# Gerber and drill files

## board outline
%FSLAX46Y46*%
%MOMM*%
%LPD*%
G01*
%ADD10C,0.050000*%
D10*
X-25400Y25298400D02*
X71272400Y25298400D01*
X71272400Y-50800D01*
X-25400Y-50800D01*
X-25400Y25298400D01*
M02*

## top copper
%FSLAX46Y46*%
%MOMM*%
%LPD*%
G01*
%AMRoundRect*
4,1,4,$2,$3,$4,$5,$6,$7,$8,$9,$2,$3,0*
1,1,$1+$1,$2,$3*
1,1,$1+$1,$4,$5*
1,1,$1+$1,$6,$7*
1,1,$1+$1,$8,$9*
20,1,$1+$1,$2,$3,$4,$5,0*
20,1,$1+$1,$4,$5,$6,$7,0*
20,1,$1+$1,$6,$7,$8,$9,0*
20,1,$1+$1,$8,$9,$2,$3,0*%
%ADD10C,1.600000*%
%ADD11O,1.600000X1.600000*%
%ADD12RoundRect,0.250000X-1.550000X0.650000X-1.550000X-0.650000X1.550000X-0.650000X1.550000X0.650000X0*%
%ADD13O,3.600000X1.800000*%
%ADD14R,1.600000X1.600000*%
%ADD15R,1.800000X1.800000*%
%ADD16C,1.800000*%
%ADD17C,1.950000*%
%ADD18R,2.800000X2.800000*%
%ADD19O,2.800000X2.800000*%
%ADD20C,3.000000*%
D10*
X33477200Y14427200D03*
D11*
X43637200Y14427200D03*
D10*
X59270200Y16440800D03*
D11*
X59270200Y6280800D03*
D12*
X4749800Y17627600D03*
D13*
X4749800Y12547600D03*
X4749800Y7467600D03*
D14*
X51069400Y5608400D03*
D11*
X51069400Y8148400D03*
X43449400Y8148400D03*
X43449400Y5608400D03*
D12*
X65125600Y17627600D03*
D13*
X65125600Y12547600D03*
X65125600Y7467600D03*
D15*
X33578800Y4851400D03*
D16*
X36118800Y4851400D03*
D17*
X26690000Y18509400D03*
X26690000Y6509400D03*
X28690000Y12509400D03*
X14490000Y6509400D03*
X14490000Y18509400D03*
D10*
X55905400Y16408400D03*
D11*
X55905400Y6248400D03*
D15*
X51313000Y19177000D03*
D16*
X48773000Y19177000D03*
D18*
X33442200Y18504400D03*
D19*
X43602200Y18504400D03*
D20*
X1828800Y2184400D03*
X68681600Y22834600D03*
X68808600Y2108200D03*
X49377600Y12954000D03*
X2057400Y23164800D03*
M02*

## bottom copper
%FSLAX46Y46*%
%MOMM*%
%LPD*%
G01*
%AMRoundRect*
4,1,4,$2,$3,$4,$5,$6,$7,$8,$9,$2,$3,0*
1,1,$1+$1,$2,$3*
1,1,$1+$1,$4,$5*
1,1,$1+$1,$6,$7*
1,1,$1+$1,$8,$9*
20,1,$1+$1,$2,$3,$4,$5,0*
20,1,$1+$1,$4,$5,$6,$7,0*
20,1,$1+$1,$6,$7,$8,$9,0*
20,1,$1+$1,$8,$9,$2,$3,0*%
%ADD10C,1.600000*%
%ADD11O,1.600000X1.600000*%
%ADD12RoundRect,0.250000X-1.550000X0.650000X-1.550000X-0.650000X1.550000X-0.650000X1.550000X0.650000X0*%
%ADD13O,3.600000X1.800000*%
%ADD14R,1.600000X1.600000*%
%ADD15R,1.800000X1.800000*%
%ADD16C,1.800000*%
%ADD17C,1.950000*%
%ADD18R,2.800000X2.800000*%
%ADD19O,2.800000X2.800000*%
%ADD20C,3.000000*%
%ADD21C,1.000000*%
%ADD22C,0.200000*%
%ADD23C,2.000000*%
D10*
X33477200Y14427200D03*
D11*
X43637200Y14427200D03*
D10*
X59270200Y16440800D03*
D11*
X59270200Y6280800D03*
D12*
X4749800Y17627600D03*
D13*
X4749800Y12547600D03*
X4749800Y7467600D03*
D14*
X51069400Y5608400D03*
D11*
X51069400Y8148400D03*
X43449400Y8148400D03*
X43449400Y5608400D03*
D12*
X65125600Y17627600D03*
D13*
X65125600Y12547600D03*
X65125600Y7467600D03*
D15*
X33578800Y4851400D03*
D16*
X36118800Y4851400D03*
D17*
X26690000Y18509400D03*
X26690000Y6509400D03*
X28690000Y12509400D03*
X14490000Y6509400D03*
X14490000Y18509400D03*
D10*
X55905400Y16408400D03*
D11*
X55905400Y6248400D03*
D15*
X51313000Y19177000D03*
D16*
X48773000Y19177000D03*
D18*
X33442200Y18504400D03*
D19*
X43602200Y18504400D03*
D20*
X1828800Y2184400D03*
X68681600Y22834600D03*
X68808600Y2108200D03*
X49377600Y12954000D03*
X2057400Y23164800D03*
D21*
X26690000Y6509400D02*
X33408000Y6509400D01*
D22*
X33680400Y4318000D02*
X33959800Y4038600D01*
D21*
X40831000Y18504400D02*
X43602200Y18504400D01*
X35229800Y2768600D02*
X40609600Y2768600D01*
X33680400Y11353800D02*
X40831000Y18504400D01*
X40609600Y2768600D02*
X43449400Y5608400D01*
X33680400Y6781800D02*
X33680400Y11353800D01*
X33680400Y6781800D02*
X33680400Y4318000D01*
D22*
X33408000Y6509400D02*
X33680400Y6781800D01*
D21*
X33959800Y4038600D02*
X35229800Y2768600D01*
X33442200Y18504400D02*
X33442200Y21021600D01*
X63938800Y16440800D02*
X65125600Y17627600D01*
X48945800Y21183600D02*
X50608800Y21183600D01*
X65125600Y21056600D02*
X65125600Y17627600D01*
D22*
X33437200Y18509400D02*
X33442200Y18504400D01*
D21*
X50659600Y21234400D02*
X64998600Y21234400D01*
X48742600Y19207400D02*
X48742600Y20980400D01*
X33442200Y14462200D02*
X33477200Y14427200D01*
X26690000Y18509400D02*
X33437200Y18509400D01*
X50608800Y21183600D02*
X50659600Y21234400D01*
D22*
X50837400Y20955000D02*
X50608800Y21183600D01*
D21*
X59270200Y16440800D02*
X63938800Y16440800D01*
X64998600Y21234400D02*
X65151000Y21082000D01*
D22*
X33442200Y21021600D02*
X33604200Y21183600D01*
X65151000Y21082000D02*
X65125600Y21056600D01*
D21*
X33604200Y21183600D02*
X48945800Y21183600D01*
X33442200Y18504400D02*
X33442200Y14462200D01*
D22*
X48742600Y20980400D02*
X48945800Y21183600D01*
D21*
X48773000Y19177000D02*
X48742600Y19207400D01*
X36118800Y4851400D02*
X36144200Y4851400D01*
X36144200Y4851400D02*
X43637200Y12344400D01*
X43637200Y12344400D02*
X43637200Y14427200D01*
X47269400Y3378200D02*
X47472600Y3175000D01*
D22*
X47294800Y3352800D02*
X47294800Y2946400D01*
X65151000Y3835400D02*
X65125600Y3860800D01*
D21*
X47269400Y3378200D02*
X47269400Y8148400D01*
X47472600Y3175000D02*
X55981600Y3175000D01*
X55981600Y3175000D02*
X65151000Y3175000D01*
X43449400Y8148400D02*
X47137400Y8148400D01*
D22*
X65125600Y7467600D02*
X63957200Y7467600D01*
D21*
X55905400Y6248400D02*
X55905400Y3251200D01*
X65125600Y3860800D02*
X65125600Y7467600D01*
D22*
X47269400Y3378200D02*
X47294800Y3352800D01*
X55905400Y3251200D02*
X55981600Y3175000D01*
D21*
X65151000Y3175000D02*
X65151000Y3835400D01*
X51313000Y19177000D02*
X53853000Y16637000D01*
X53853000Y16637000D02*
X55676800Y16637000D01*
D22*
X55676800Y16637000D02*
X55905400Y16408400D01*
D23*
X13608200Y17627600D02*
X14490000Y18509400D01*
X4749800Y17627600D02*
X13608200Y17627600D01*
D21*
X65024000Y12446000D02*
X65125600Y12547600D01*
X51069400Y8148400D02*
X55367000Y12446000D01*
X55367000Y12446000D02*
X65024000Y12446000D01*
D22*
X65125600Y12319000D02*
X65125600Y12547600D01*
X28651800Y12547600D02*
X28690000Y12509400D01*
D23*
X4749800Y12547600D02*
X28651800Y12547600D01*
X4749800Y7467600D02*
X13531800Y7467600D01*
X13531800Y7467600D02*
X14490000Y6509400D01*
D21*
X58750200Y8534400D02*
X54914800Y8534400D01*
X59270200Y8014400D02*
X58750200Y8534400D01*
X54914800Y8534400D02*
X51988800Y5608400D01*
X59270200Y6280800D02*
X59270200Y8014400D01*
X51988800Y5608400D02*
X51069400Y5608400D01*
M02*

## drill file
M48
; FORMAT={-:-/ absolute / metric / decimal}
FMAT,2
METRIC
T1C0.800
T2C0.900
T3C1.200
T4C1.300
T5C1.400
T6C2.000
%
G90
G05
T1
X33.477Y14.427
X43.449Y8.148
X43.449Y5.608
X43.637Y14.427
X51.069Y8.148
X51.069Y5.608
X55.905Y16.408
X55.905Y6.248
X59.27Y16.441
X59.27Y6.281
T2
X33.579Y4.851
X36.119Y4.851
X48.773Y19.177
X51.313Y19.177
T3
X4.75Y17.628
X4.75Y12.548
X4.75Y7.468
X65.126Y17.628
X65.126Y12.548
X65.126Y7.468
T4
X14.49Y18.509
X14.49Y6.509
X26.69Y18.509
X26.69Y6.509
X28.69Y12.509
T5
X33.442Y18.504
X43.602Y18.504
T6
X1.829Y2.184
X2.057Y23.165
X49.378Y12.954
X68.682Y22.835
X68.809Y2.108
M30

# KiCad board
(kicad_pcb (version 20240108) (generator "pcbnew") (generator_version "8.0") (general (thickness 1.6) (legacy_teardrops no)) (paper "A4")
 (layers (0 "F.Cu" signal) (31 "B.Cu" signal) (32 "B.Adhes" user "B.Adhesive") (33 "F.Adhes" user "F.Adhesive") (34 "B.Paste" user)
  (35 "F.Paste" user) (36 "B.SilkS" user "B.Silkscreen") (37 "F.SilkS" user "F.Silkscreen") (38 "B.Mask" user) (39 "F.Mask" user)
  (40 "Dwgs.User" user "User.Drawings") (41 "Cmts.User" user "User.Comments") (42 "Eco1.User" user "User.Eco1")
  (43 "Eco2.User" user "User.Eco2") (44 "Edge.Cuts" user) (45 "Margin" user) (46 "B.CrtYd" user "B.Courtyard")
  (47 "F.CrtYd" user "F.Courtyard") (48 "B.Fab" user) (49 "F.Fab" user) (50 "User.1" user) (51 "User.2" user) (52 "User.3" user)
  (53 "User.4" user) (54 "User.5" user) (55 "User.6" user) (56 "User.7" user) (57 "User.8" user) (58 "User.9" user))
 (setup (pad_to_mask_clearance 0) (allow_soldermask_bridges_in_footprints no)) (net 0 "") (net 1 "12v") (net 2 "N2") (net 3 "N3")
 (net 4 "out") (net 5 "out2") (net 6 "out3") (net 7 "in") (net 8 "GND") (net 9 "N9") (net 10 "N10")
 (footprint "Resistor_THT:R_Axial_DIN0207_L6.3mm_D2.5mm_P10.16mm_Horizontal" (layer "F.Cu") (at 33.4772 -14.4272)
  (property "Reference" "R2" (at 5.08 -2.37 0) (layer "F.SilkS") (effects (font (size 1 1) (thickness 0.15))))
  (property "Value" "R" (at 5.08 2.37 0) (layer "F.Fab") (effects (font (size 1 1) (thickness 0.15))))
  (pad "1" thru_hole circle (at 0 0) (size 1.6 1.6) (drill 0.8) (layers "*.Cu" "*.Mask") (remove_unused_layers no) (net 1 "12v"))
  (pad "2" thru_hole oval (at 10.16 0) (size 1.6 1.6) (drill 0.8) (layers "*.Cu" "*.Mask") (remove_unused_layers no) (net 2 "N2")))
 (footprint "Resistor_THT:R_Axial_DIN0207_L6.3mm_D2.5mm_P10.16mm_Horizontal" (layer "F.Cu") (at 59.2702 -16.4408 -90)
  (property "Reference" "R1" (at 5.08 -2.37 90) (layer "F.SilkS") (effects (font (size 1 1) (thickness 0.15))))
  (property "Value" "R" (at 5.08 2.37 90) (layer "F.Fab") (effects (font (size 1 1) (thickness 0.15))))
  (pad "1" thru_hole circle (at 0 0 270) (size 1.6 1.6) (drill 0.8) (layers "*.Cu" "*.Mask") (remove_unused_layers no) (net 1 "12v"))
  (pad "2" thru_hole oval (at 10.16 0 270) (size 1.6 1.6) (drill 0.8) (layers "*.Cu" "*.Mask") (remove_unused_layers no) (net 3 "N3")))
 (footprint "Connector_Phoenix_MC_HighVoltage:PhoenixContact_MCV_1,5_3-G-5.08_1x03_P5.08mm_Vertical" (layer "F.Cu") (at 4.7498 -17.6276 -90)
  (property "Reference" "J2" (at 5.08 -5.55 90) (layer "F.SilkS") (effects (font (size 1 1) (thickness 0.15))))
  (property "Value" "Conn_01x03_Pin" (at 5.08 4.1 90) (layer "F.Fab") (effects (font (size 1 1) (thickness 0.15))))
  (pad "1" thru_hole roundrect (at 0 0 270) (size 1.8 3.6) (drill 1.2) (layers "*.Cu" "*.Mask") (remove_unused_layers no)
   (roundrect_rratio 0.138889) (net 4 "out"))
  (pad "2" thru_hole oval (at 5.08 0 270) (size 1.8 3.6) (drill 1.2) (layers "*.Cu" "*.Mask") (remove_unused_layers no) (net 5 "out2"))
  (pad "3" thru_hole oval (at 10.16 0 270) (size 1.8 3.6) (drill 1.2) (layers "*.Cu" "*.Mask") (remove_unused_layers no) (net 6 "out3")))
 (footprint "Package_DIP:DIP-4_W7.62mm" (layer "F.Cu") (at 51.0694 -5.6084 180)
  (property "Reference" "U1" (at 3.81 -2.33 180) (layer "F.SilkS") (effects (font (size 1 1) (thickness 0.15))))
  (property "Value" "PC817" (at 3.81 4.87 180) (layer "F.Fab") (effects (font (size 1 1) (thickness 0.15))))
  (pad "1" thru_hole rect (at 0 0 180) (size 1.6 1.6) (drill 0.8) (layers "*.Cu" "*.Mask") (remove_unused_layers no) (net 3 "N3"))
  (pad "2" thru_hole oval (at 0 2.54 180) (size 1.6 1.6) (drill 0.8) (layers "*.Cu" "*.Mask") (remove_unused_layers no) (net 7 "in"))
  (pad "3" thru_hole oval (at 7.62 2.54 180) (size 1.6 1.6) (drill 0.8) (layers "*.Cu" "*.Mask") (remove_unused_layers no) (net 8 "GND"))
  (pad "4" thru_hole oval (at 7.62 0 180) (size 1.6 1.6) (drill 0.8) (layers "*.Cu" "*.Mask") (remove_unused_layers no) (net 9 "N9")))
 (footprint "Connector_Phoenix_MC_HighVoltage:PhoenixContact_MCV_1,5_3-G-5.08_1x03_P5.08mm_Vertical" (layer "F.Cu")
  (at 65.1256 -17.6276 -90)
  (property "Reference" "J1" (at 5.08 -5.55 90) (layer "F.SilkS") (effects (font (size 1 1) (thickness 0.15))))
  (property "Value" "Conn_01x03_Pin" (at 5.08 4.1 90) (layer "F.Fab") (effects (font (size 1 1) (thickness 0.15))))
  (pad "1" thru_hole roundrect (at 0 0 270) (size 1.8 3.6) (drill 1.2) (layers "*.Cu" "*.Mask") (remove_unused_layers no)
   (roundrect_rratio 0.138889) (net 1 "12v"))
  (pad "2" thru_hole oval (at 5.08 0 270) (size 1.8 3.6) (drill 1.2) (layers "*.Cu" "*.Mask") (remove_unused_layers no) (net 7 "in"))
  (pad "3" thru_hole oval (at 10.16 0 270) (size 1.8 3.6) (drill 1.2) (layers "*.Cu" "*.Mask") (remove_unused_layers no) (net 8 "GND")))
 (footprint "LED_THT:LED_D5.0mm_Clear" (layer "F.Cu") (at 33.5788 -4.8514)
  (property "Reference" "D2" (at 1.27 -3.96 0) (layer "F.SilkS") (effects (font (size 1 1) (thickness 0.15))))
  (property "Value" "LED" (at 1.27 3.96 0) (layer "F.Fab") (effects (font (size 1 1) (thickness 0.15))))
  (pad "1" thru_hole rect (at 0 0) (size 1.8 1.8) (drill 0.9) (layers "*.Cu" "*.Mask") (remove_unused_layers no) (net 9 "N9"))
  (pad "2" thru_hole circle (at 2.54 0) (size 1.8 1.8) (drill 0.9) (layers "*.Cu" "*.Mask") (remove_unused_layers no) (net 2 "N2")))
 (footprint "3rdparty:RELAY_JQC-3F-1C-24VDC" (layer "F.Cu") (at 20.59 -12.5094)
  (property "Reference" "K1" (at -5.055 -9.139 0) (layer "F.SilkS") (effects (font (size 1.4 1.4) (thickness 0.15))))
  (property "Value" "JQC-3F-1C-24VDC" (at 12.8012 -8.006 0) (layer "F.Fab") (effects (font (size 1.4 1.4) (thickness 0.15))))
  (pad "COIL1" thru_hole circle (at 6.1 -6) (size 1.95 1.95) (drill 1.3) (layers "*.Cu" "*.Mask") (remove_unused_layers no) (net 1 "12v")
   (solder_mask_margin 0.102))
  (pad "COIL2" thru_hole circle (at 6.1 6) (size 1.95 1.95) (drill 1.3) (layers "*.Cu" "*.Mask") (remove_unused_layers no) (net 9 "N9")
   (solder_mask_margin 0.102))
  (pad "COM" thru_hole circle (at 8.1 0) (size 1.95 1.95) (drill 1.3) (layers "*.Cu" "*.Mask") (remove_unused_layers no) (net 5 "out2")
   (solder_mask_margin 0.102))
  (pad "NC" thru_hole circle (at -6.1 6) (size 1.95 1.95) (drill 1.3) (layers "*.Cu" "*.Mask") (remove_unused_layers no) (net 6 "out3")
   (solder_mask_margin 0.102))
  (pad "NO" thru_hole circle (at -6.1 -6) (size 1.95 1.95) (drill 1.3) (layers "*.Cu" "*.Mask") (remove_unused_layers no) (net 4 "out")
   (solder_mask_margin 0.102)))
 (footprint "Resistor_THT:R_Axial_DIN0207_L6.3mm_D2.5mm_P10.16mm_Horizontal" (layer "F.Cu") (at 55.9054 -16.4084 -90)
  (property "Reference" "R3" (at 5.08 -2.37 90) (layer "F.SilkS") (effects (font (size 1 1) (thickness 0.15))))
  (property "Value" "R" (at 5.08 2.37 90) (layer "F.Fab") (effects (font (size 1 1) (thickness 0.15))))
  (pad "1" thru_hole circle (at 0 0 270) (size 1.6 1.6) (drill 0.8) (layers "*.Cu" "*.Mask") (remove_unused_layers no) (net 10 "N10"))
  (pad "2" thru_hole oval (at 10.16 0 270) (size 1.6 1.6) (drill 0.8) (layers "*.Cu" "*.Mask") (remove_unused_layers no) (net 8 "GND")))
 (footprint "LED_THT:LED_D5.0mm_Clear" (layer "F.Cu") (at 51.313 -19.177 180)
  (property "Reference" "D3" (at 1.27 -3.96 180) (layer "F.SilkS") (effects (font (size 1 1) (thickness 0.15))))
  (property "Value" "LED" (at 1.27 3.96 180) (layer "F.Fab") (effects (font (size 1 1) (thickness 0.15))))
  (pad "1" thru_hole rect (at 0 0 180) (size 1.8 1.8) (drill 0.9) (layers "*.Cu" "*.Mask") (remove_unused_layers no) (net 10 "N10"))
  (pad "2" thru_hole circle (at 2.54 0 180) (size 1.8 1.8) (drill 0.9) (layers "*.Cu" "*.Mask") (remove_unused_layers no) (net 1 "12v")))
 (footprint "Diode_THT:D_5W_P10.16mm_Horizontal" (layer "F.Cu") (at 33.4422 -18.5044)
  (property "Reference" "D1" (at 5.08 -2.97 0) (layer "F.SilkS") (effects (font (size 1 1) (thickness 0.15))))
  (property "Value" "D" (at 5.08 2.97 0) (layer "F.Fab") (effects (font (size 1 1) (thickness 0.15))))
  (pad "1" thru_hole rect (at 0 0) (size 2.8 2.8) (drill 1.4) (layers "*.Cu" "*.Mask") (remove_unused_layers no) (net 1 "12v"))
  (pad "2" thru_hole oval (at 10.16 0) (size 2.8 2.8) (drill 1.4) (layers "*.Cu" "*.Mask") (remove_unused_layers no) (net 9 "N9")))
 (gr_rect (start -0.0254 -25.2984) (end 71.2724 0.0508) (stroke (width 0.05) (type default)) (fill none) (layer "Edge.Cuts"))
 (via (at 1.8288 -2.1844) (size 3) (drill 2) (layers "F.Cu" "B.Cu") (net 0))
 (via (at 68.6816 -22.8346) (size 3) (drill 2) (layers "F.Cu" "B.Cu") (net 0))
 (via (at 68.8086 -2.1082) (size 3) (drill 2) (layers "F.Cu" "B.Cu") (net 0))
 (via (at 49.3776 -12.954) (size 3) (drill 2) (layers "F.Cu" "B.Cu") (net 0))
 (via (at 2.0574 -23.1648) (size 3) (drill 2) (layers "F.Cu" "B.Cu") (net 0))
 (segment (start 26.69 -6.5094) (end 33.408 -6.5094) (width 1) (layer "B.Cu") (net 9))
 (segment (start 33.6804 -4.318) (end 33.9598 -4.0386) (width 0.2) (layer "B.Cu") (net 9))
 (segment (start 40.831 -18.5044) (end 43.6022 -18.5044) (width 1) (layer "B.Cu") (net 9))
 (segment (start 35.2298 -2.7686) (end 40.6096 -2.7686) (width 1) (layer "B.Cu") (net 9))
 (segment (start 33.6804 -11.3538) (end 40.831 -18.5044) (width 1) (layer "B.Cu") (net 9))
 (segment (start 40.6096 -2.7686) (end 43.4494 -5.6084) (width 1) (layer "B.Cu") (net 9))
 (segment (start 33.6804 -6.7818) (end 33.6804 -11.3538) (width 1) (layer "B.Cu") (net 9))
 (segment (start 33.6804 -6.7818) (end 33.6804 -4.318) (width 1) (layer "B.Cu") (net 9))
 (segment (start 33.408 -6.5094) (end 33.6804 -6.7818) (width 0.2) (layer "B.Cu") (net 9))
 (segment (start 33.9598 -4.0386) (end 35.2298 -2.7686) (width 1) (layer "B.Cu") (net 9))
 (segment (start 33.4422 -18.5044) (end 33.4422 -21.0216) (width 1) (layer "B.Cu") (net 1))
 (segment (start 63.9388 -16.4408) (end 65.1256 -17.6276) (width 1) (layer "B.Cu") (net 1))
 (segment (start 48.9458 -21.1836) (end 50.6088 -21.1836) (width 1) (layer "B.Cu") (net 1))
 (segment (start 65.1256 -21.0566) (end 65.1256 -17.6276) (width 1) (layer "B.Cu") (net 1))
 (segment (start 33.4372 -18.5094) (end 33.4422 -18.5044) (width 0.2) (layer "B.Cu") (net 1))
 (segment (start 50.6596 -21.2344) (end 64.9986 -21.2344) (width 1) (layer "B.Cu") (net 1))
 (segment (start 48.7426 -19.2074) (end 48.7426 -20.9804) (width 1) (layer "B.Cu") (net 1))
 (segment (start 33.4422 -14.4622) (end 33.4772 -14.4272) (width 1) (layer "B.Cu") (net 1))
 (segment (start 26.69 -18.5094) (end 33.4372 -18.5094) (width 1) (layer "B.Cu") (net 1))
 (segment (start 50.6088 -21.1836) (end 50.6596 -21.2344) (width 1) (layer "B.Cu") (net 1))
 (segment (start 50.8374 -20.955) (end 50.6088 -21.1836) (width 0.2) (layer "B.Cu") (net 1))
 (segment (start 59.2702 -16.4408) (end 63.9388 -16.4408) (width 1) (layer "B.Cu") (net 1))
 (segment (start 64.9986 -21.2344) (end 65.151 -21.082) (width 1) (layer "B.Cu") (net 1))
 (segment (start 33.4422 -21.0216) (end 33.6042 -21.1836) (width 0.2) (layer "B.Cu") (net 1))
 (segment (start 65.151 -21.082) (end 65.1256 -21.0566) (width 0.2) (layer "B.Cu") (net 1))
 (segment (start 33.6042 -21.1836) (end 48.9458 -21.1836) (width 1) (layer "B.Cu") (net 1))
 (segment (start 33.4422 -18.5044) (end 33.4422 -14.4622) (width 1) (layer "B.Cu") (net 1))
 (segment (start 48.7426 -20.9804) (end 48.9458 -21.1836) (width 0.2) (layer "B.Cu") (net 1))
 (segment (start 48.773 -19.177) (end 48.7426 -19.2074) (width 1) (layer "B.Cu") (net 1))
 (segment (start 36.1188 -4.8514) (end 36.1442 -4.8514) (width 1) (layer "B.Cu") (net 2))
 (segment (start 36.1442 -4.8514) (end 43.6372 -12.3444) (width 1) (layer "B.Cu") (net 2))
 (segment (start 43.6372 -12.3444) (end 43.6372 -14.4272) (width 1) (layer "B.Cu") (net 2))
 (segment (start 47.2694 -3.3782) (end 47.4726 -3.175) (width 1) (layer "B.Cu") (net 8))
 (segment (start 47.2948 -3.3528) (end 47.2948 -2.9464) (width 0.2) (layer "B.Cu") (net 8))
 (segment (start 65.151 -3.8354) (end 65.1256 -3.8608) (width 0.2) (layer "B.Cu") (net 8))
 (segment (start 47.2694 -3.3782) (end 47.2694 -8.1484) (width 1) (layer "B.Cu") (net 8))
 (segment (start 47.4726 -3.175) (end 55.9816 -3.175) (width 1) (layer "B.Cu") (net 8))
 (segment (start 55.9816 -3.175) (end 65.151 -3.175) (width 1) (layer "B.Cu") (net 8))
 (segment (start 43.4494 -8.1484) (end 47.1374 -8.1484) (width 1) (layer "B.Cu") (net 8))
 (segment (start 65.1256 -7.4676) (end 63.9572 -7.4676) (width 0.2) (layer "B.Cu") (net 8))
 (segment (start 55.9054 -6.2484) (end 55.9054 -3.2512) (width 1) (layer "B.Cu") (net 8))
 (segment (start 65.1256 -3.8608) (end 65.1256 -7.4676) (width 1) (layer "B.Cu") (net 8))
 (segment (start 47.2694 -3.3782) (end 47.2948 -3.3528) (width 0.2) (layer "B.Cu") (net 8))
 (segment (start 55.9054 -3.2512) (end 55.9816 -3.175) (width 0.2) (layer "B.Cu") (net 8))
 (segment (start 65.151 -3.175) (end 65.151 -3.8354) (width 1) (layer "B.Cu") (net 8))
 (segment (start 51.313 -19.177) (end 53.853 -16.637) (width 1) (layer "B.Cu") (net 10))
 (segment (start 53.853 -16.637) (end 55.6768 -16.637) (width 1) (layer "B.Cu") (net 10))
 (segment (start 55.6768 -16.637) (end 55.9054 -16.4084) (width 0.2) (layer "B.Cu") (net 10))
 (segment (start 13.6082 -17.6276) (end 14.49 -18.5094) (width 2) (layer "B.Cu") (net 4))
 (segment (start 4.7498 -17.6276) (end 13.6082 -17.6276) (width 2) (layer "B.Cu") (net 4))
 (segment (start 65.024 -12.446) (end 65.1256 -12.5476) (width 1) (layer "B.Cu") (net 7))
 (segment (start 51.0694 -8.1484) (end 55.367 -12.446) (width 1) (layer "B.Cu") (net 7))
 (segment (start 55.367 -12.446) (end 65.024 -12.446) (width 1) (layer "B.Cu") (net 7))
 (segment (start 65.1256 -12.319) (end 65.1256 -12.5476) (width 0.2) (layer "B.Cu") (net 7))
 (segment (start 28.6518 -12.5476) (end 28.69 -12.5094) (width 0.2) (layer "B.Cu") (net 5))
 (segment (start 4.7498 -12.5476) (end 28.6518 -12.5476) (width 2) (layer "B.Cu") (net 5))
 (segment (start 4.7498 -7.4676) (end 13.5318 -7.4676) (width 2) (layer "B.Cu") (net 6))
 (segment (start 13.5318 -7.4676) (end 14.49 -6.5094) (width 2) (layer "B.Cu") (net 6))
 (segment (start 58.7502 -8.5344) (end 54.9148 -8.5344) (width 1) (layer "B.Cu") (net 3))
 (segment (start 59.2702 -8.0144) (end 58.7502 -8.5344) (width 1) (layer "B.Cu") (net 3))
 (segment (start 54.9148 -8.5344) (end 51.9888 -5.6084) (width 1) (layer "B.Cu") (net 3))
 (segment (start 59.2702 -6.2808) (end 59.2702 -8.0144) (width 1) (layer "B.Cu") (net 3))
 (segment (start 51.9888 -5.6084) (end 51.0694 -5.6084) (width 1) (layer "B.Cu") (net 3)))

